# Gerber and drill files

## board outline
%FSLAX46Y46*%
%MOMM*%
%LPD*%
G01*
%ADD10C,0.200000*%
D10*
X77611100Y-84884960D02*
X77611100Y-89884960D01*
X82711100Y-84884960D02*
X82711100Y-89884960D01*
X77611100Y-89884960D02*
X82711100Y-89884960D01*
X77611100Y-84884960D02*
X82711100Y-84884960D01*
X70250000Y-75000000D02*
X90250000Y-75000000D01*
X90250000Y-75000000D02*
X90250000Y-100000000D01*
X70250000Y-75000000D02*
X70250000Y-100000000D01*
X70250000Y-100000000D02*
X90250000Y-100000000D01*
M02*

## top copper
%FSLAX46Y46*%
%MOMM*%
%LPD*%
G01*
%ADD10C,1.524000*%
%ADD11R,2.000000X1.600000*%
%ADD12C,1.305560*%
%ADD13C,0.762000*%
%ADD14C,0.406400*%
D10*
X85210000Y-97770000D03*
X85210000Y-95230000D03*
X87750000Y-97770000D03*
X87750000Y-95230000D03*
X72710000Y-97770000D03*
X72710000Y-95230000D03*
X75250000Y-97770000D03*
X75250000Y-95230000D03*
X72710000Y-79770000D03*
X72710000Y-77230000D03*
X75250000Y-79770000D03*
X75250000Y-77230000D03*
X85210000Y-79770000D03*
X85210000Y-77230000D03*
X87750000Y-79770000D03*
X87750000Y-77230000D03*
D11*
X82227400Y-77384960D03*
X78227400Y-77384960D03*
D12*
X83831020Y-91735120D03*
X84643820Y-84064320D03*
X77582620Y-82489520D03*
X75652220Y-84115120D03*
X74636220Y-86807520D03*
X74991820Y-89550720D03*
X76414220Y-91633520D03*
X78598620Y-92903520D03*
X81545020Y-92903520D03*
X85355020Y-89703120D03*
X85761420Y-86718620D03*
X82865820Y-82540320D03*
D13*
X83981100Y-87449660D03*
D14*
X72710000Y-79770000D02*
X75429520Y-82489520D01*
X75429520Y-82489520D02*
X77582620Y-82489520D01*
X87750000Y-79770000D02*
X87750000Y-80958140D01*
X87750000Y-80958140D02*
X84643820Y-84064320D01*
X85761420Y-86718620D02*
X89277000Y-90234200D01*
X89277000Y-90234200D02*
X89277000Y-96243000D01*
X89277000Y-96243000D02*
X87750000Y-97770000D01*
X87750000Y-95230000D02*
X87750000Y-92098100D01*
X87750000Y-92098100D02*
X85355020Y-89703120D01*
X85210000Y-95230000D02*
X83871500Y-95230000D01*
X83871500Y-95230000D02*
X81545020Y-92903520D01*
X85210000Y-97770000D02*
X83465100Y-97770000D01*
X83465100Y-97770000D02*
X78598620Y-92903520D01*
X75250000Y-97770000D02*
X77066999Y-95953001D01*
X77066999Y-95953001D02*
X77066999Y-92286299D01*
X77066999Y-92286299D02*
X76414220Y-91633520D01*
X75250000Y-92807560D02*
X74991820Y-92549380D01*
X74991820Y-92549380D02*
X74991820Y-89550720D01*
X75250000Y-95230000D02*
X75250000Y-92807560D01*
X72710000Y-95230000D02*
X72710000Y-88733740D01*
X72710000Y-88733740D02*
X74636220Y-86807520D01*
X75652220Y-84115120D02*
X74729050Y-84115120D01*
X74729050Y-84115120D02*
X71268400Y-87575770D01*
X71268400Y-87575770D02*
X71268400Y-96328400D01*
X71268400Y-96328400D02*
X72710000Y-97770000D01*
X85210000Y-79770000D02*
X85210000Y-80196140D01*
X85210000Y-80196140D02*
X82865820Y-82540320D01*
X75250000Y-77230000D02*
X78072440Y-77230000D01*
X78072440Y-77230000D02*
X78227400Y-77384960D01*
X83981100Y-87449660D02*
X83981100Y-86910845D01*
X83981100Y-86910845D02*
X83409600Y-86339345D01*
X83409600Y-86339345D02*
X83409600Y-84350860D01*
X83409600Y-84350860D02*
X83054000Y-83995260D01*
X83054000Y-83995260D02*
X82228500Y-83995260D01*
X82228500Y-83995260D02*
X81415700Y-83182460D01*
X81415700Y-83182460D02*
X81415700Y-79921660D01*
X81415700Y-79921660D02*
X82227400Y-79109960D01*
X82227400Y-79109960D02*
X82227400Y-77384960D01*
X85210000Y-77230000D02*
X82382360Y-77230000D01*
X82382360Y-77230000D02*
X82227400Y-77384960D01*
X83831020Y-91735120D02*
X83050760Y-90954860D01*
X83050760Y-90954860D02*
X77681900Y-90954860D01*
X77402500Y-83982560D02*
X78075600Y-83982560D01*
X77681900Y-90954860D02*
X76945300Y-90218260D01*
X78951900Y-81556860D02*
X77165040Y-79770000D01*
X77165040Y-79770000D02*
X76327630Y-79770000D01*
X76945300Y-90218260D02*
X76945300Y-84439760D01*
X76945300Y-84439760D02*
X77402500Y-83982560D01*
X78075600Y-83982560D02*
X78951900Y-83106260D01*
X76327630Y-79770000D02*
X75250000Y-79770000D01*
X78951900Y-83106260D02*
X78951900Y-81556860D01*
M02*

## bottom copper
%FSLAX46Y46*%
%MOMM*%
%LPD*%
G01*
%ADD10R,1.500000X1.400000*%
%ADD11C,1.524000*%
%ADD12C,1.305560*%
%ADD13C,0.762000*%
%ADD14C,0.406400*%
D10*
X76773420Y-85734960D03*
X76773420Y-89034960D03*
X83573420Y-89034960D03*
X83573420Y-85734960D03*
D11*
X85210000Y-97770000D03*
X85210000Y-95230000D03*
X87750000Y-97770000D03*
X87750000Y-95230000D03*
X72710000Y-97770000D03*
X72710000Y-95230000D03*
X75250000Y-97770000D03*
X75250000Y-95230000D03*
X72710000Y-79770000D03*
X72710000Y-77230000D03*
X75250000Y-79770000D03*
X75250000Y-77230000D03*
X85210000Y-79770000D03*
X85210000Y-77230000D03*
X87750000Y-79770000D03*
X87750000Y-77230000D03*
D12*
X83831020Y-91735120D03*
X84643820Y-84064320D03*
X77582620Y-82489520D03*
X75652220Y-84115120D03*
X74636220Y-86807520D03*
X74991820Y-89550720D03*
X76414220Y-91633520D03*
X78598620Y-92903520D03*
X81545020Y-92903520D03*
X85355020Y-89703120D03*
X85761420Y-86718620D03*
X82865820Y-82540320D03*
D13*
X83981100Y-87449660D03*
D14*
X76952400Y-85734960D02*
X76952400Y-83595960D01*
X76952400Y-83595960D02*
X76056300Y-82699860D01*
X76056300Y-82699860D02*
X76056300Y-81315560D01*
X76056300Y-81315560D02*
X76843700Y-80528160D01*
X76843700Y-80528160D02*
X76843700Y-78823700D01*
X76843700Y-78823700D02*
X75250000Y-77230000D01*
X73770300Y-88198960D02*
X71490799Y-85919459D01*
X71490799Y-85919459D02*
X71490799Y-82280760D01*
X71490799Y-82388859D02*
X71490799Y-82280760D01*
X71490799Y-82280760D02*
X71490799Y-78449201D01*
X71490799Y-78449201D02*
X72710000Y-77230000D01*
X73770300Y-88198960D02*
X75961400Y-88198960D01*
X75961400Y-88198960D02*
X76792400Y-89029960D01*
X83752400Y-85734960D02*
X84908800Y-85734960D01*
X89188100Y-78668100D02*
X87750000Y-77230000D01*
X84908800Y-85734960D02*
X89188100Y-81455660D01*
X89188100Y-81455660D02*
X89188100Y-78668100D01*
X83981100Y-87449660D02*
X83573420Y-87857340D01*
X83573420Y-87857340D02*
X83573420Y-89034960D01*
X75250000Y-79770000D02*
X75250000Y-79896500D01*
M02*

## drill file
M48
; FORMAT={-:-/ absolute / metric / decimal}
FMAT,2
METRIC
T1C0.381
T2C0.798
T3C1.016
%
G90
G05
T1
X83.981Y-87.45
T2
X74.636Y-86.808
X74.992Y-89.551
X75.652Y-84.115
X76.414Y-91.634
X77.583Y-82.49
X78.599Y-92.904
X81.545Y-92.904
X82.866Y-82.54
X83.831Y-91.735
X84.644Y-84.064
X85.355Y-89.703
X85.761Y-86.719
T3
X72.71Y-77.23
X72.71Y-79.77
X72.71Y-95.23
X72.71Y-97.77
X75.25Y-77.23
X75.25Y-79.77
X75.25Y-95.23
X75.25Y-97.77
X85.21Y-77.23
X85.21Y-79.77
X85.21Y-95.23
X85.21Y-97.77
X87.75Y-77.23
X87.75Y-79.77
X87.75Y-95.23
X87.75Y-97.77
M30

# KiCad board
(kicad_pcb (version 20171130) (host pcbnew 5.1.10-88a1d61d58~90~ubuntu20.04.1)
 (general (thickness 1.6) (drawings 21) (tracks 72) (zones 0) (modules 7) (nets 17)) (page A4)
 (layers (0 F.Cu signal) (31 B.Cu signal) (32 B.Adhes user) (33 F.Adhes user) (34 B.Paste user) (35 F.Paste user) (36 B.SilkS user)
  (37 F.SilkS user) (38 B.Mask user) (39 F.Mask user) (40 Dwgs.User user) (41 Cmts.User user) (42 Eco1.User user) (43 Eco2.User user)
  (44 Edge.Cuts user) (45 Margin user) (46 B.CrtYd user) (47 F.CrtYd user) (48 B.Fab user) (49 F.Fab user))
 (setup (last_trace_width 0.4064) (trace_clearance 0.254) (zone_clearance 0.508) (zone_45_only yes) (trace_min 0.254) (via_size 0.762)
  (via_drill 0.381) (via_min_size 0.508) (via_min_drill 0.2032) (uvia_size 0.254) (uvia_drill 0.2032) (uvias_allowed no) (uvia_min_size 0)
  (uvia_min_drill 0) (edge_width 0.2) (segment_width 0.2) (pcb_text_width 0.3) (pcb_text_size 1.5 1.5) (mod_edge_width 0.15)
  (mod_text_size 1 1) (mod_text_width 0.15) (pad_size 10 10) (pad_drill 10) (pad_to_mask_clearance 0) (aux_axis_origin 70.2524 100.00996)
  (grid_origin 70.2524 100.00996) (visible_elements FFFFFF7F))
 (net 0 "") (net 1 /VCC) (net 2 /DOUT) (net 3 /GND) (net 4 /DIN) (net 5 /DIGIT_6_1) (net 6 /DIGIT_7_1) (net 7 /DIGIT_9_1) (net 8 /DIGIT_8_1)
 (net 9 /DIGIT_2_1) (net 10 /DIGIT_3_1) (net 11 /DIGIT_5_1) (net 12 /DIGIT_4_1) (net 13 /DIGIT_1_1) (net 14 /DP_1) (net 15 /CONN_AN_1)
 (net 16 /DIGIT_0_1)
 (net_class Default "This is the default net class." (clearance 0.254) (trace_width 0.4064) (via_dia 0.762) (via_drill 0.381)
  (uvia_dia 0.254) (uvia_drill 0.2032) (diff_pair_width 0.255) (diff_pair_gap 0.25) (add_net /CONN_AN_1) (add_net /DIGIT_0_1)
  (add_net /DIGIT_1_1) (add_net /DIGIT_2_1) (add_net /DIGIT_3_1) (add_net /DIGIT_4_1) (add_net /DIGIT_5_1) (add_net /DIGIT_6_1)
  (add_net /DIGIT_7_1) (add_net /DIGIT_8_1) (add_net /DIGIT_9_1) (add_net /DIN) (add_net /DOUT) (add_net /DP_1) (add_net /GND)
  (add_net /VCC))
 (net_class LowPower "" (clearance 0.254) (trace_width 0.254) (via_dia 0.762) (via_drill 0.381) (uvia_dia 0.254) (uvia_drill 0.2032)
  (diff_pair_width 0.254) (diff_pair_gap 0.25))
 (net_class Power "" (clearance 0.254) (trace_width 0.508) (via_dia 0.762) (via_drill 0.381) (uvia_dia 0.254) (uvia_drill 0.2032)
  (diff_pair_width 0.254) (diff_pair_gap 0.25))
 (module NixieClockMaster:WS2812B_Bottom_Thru (layer F.Cu) (at 80.17342 87.38496 90)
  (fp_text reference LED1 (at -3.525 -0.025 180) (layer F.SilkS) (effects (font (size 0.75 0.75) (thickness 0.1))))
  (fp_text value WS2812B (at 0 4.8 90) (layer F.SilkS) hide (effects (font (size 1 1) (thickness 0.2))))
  (pad 1 smd rect (at 1.65 -3.4 90) (size 1.4 1.5) (layers B.Cu B.Paste B.Mask) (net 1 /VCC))
  (pad 2 smd rect (at -1.65 -3.4 90) (size 1.4 1.5) (layers B.Cu B.Paste B.Mask) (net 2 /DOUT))
  (pad 3 smd rect (at -1.65 3.4 90) (size 1.4 1.5) (layers B.Cu B.Paste B.Mask) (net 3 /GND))
  (pad 4 smd rect (at 1.65 3.4 90) (size 1.4 1.5) (layers B.Cu B.Paste B.Mask) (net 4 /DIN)))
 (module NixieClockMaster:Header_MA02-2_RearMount (layer F.Cu) (at 87.75 96.5)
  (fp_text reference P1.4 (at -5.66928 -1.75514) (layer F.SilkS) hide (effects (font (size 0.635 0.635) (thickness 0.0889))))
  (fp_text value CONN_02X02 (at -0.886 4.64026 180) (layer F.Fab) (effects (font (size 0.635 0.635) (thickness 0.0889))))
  (pad 1 thru_hole circle (at -2.54 1.27) (size 1.524 1.524) (drill 1.016) (layers *.Cu *.Mask F.Paste F.SilkS) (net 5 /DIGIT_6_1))
  (pad 2 thru_hole circle (at -2.54 -1.27) (size 1.524 1.524) (drill 1.016) (layers *.Cu *.Mask F.Paste F.SilkS) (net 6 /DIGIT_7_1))
  (pad 3 thru_hole circle (at 0 1.27) (size 1.524 1.524) (drill 1.016) (layers *.Cu *.Mask F.Paste F.SilkS) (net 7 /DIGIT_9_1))
  (pad 4 thru_hole circle (at 0 -1.27) (size 1.524 1.524) (drill 1.016) (layers *.Cu *.Mask F.Paste F.SilkS) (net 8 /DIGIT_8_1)))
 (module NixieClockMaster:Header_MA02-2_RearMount (layer F.Cu) (at 75.25 96.5)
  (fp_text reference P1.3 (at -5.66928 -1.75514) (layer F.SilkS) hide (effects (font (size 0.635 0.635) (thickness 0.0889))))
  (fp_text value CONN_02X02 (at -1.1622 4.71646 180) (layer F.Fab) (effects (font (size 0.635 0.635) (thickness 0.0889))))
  (pad 1 thru_hole circle (at -2.54 1.27) (size 1.524 1.524) (drill 1.016) (layers *.Cu *.Mask F.Paste F.SilkS) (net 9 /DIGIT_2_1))
  (pad 2 thru_hole circle (at -2.54 -1.27) (size 1.524 1.524) (drill 1.016) (layers *.Cu *.Mask F.Paste F.SilkS) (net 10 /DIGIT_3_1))
  (pad 3 thru_hole circle (at 0 1.27) (size 1.524 1.524) (drill 1.016) (layers *.Cu *.Mask F.Paste F.SilkS) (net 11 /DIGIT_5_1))
  (pad 4 thru_hole circle (at 0 -1.27) (size 1.524 1.524) (drill 1.016) (layers *.Cu *.Mask F.Paste F.SilkS) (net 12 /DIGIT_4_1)))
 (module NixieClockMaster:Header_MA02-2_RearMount (layer F.Cu) (at 75.25 78.5)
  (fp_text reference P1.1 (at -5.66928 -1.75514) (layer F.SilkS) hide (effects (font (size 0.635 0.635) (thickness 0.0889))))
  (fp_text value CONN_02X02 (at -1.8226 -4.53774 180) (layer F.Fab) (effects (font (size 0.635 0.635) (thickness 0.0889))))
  (pad 1 thru_hole circle (at -2.54 1.27) (size 1.524 1.524) (drill 1.016) (layers *.Cu *.Mask F.Paste F.SilkS) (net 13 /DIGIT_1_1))
  (pad 2 thru_hole circle (at -2.54 -1.27) (size 1.524 1.524) (drill 1.016) (layers *.Cu *.Mask F.Paste F.SilkS) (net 2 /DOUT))
  (pad 3 thru_hole circle (at 0 1.27) (size 1.524 1.524) (drill 1.016) (layers *.Cu *.Mask F.Paste F.SilkS) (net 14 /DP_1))
  (pad 4 thru_hole circle (at 0 -1.27) (size 1.524 1.524) (drill 1.016) (layers *.Cu *.Mask F.Paste F.SilkS) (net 1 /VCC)))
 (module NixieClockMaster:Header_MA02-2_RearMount (layer F.Cu) (at 87.75 78.5)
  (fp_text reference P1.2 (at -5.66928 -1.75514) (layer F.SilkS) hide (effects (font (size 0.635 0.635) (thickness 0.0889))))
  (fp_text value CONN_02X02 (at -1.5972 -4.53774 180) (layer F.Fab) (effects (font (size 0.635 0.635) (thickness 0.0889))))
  (pad 1 thru_hole circle (at -2.54 1.27) (size 1.524 1.524) (drill 1.016) (layers *.Cu *.Mask F.Paste F.SilkS) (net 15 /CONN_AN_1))
  (pad 2 thru_hole circle (at -2.54 -1.27) (size 1.524 1.524) (drill 1.016) (layers *.Cu *.Mask F.Paste F.SilkS) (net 3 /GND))
  (pad 3 thru_hole circle (at 0 1.27) (size 1.524 1.524) (drill 1.016) (layers *.Cu *.Mask F.Paste F.SilkS) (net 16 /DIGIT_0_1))
  (pad 4 thru_hole circle (at 0 -1.27) (size 1.524 1.524) (drill 1.016) (layers *.Cu *.Mask F.Paste F.SilkS) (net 4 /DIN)))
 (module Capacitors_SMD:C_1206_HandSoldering (layer F.Cu) (at 80.2274 77.38496 180)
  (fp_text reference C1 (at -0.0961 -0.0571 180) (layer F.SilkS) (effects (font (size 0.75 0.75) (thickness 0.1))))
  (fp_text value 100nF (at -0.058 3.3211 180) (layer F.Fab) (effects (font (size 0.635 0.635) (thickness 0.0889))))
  (pad 1 smd rect (at -2 0 180) (size 2 1.6) (layers F.Cu F.Paste F.Mask) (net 3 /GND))
  (pad 2 smd rect (at 2 0 180) (size 2 1.6) (layers F.Cu F.Paste F.Mask) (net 1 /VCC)))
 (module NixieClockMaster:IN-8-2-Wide (layer F.Cu) (at 80.17342 87.46792 180)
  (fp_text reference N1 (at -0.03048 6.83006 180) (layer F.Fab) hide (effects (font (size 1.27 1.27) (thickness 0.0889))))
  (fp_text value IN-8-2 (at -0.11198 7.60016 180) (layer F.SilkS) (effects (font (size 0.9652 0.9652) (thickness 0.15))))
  (pad . thru_hole circle (at -3.6576 -4.2672 180) (size 1.30556 1.30556) (drill 0.79756) (layers *.Cu *.Mask F.Paste F.SilkS)
   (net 14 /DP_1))
  (pad 0 thru_hole circle (at -4.4704 3.4036 180) (size 1.30556 1.30556) (drill 0.79756) (layers *.Cu *.Mask F.Paste F.SilkS)
   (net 16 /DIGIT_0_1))
  (pad 1 thru_hole circle (at 2.5908 4.9784 180) (size 1.30556 1.30556) (drill 0.79756) (layers *.Cu *.Mask F.Paste F.SilkS)
   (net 13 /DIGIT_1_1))
  (pad 2 thru_hole circle (at 4.5212 3.3528 180) (size 1.30556 1.30556) (drill 0.79756) (layers *.Cu *.Mask F.Paste F.SilkS)
   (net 9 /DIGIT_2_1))
  (pad 3 thru_hole circle (at 5.5372 0.6604 180) (size 1.30556 1.30556) (drill 0.79756) (layers *.Cu *.Mask F.Paste F.SilkS)
   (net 10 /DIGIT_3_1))
  (pad 4 thru_hole circle (at 5.1816 -2.0828 180) (size 1.30556 1.30556) (drill 0.79756) (layers *.Cu *.Mask F.Paste F.SilkS)
   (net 12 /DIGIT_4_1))
  (pad 5 thru_hole circle (at 3.7592 -4.1656 180) (size 1.30556 1.30556) (drill 0.79756) (layers *.Cu *.Mask F.Paste F.SilkS)
   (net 11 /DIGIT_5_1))
  (pad 6 thru_hole circle (at 1.5748 -5.4356 180) (size 1.30556 1.30556) (drill 0.79756) (layers *.Cu *.Mask F.Paste F.SilkS)
   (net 5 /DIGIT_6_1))
  (pad 7 thru_hole circle (at -1.3716 -5.4356 180) (size 1.30556 1.30556) (drill 0.79756) (layers *.Cu *.Mask F.Paste F.SilkS)
   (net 6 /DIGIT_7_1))
  (pad 8 thru_hole circle (at -5.1816 -2.2352 180) (size 1.30556 1.30556) (drill 0.79756) (layers *.Cu *.Mask F.Paste F.SilkS)
   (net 8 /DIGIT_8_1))
  (pad 9 thru_hole circle (at -5.588 0.7493 180) (size 1.30556 1.30556) (drill 0.79756) (layers *.Cu *.Mask F.Paste F.SilkS)
   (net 7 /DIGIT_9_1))
  (pad A thru_hole circle (at -2.6924 4.9276 180) (size 1.30556 1.30556) (drill 0.79756) (layers *.Cu *.Mask F.Paste F.SilkS)
   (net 15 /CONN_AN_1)))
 (gr_line (start 77.6111 84.88496) (end 77.6111 89.88496) (layer Edge.Cuts) (width 0.2))
 (gr_line (start 82.7111 84.88496) (end 82.7111 89.88496) (layer Edge.Cuts) (width 0.2))
 (gr_line (start 77.6111 89.88496) (end 82.7111 89.88496) (layer Edge.Cuts) (width 0.2))
 (gr_line (start 77.6111 84.88496) (end 82.7111 84.88496) (layer Edge.Cuts) (width 0.2))
 (gr_line (start 70.25 75) (end 90.25 75) (layer Edge.Cuts) (width 0.2))
 (gr_line (start 90.25 75) (end 90.25 100) (layer Edge.Cuts) (width 0.2))
 (gr_line (start 70.25 75) (end 70.25 100) (layer Edge.Cuts) (width 0.2))
 (gr_line (start 70.25 100) (end 90.25 100) (layer Edge.Cuts) (width 0.2))
 (segment (start 72.71 79.77) (end 75.42952 82.48952) (width 0.4064) (layer F.Cu) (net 13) (status 10))
 (segment (start 75.42952 82.48952) (end 77.58262 82.48952) (width 0.4064) (layer F.Cu) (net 13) (status 20))
 (segment (start 87.75 79.77) (end 87.75 80.95814) (width 0.4064) (layer F.Cu) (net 16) (status 10))
 (segment (start 87.75 80.95814) (end 84.64382 84.06432) (width 0.4064) (layer F.Cu) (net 16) (status 20))
 (segment (start 85.76142 86.71862) (end 89.277 90.2342) (width 0.4064) (layer F.Cu) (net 7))
 (segment (start 89.277 90.2342) (end 89.277 96.243) (width 0.4064) (layer F.Cu) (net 7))
 (segment (start 89.277 96.243) (end 87.75 97.77) (width 0.4064) (layer F.Cu) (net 7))
 (segment (start 87.75 95.23) (end 87.75 92.0981) (width 0.4064) (layer F.Cu) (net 8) (status 10))
 (segment (start 87.75 92.0981) (end 85.35502 89.70312) (width 0.4064) (layer F.Cu) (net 8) (status 20))
 (segment (start 85.21 95.23) (end 83.8715 95.23) (width 0.4064) (layer F.Cu) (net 6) (status 10))
 (segment (start 83.8715 95.23) (end 81.54502 92.90352) (width 0.4064) (layer F.Cu) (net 6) (status 20))
 (segment (start 85.21 97.77) (end 83.4651 97.77) (width 0.4064) (layer F.Cu) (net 5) (status 10))
 (segment (start 83.4651 97.77) (end 78.59862 92.90352) (width 0.4064) (layer F.Cu) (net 5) (status 20))
 (segment (start 75.25 97.77) (end 77.066999 95.953001) (width 0.4064) (layer F.Cu) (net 11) (status 10))
 (segment (start 77.066999 95.953001) (end 77.066999 92.286299) (width 0.4064) (layer F.Cu) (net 11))
 (segment (start 77.066999 92.286299) (end 76.41422 91.63352) (width 0.4064) (layer F.Cu) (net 11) (status 20))
 (segment (start 75.25 92.80756) (end 74.99182 92.54938) (width 0.4064) (layer F.Cu) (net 12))
 (segment (start 74.99182 92.54938) (end 74.99182 89.55072) (width 0.4064) (layer F.Cu) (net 12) (status 20))
 (segment (start 75.25 95.23) (end 75.25 92.80756) (width 0.4064) (layer F.Cu) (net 12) (status 10))
 (segment (start 72.71 95.23) (end 72.71 88.73374) (width 0.4064) (layer F.Cu) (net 10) (status 10))
 (segment (start 72.71 88.73374) (end 74.63622 86.80752) (width 0.4064) (layer F.Cu) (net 10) (status 20))
 (segment (start 75.65222 84.11512) (end 74.72905 84.11512) (width 0.4064) (layer F.Cu) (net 9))
 (segment (start 74.72905 84.11512) (end 71.2684 87.57577) (width 0.4064) (layer F.Cu) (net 9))
 (segment (start 71.2684 87.57577) (end 71.2684 96.3284) (width 0.4064) (layer F.Cu) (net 9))
 (segment (start 71.2684 96.3284) (end 72.71 97.77) (width 0.4064) (layer F.Cu) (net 9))
 (segment (start 85.21 79.77) (end 85.21 80.19614) (width 0.4064) (layer F.Cu) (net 15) (status 30))
 (segment (start 85.21 80.19614) (end 82.86582 82.54032) (width 0.4064) (layer F.Cu) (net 15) (status 30))
 (segment (start 76.9524 85.73496) (end 76.9524 83.59596) (width 0.4064) (layer B.Cu) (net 1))
 (segment (start 76.9524 83.59596) (end 76.0563 82.69986) (width 0.4064) (layer B.Cu) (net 1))
 (segment (start 76.0563 82.69986) (end 76.0563 81.31556) (width 0.4064) (layer B.Cu) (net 1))
 (segment (start 76.0563 81.31556) (end 76.8437 80.52816) (width 0.4064) (layer B.Cu) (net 1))
 (segment (start 76.8437 80.52816) (end 76.8437 78.8237) (width 0.4064) (layer B.Cu) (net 1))
 (segment (start 76.8437 78.8237) (end 75.25 77.23) (width 0.4064) (layer B.Cu) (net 1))
 (segment (start 75.25 77.23) (end 78.07244 77.23) (width 0.4064) (layer F.Cu) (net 1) (status 30))
 (segment (start 78.07244 77.23) (end 78.2274 77.38496) (width 0.4064) (layer F.Cu) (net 1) (status 30))
 (segment (start 73.7703 88.19896) (end 71.490799 85.919459) (width 0.4064) (layer B.Cu) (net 2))
 (segment (start 71.490799 85.919459) (end 71.490799 82.28076) (width 0.4064) (layer B.Cu) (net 2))
 (segment (start 71.490799 82.388859) (end 71.490799 82.28076) (width 0.4064) (layer B.Cu) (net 2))
 (segment (start 71.490799 82.28076) (end 71.490799 78.449201) (width 0.4064) (layer B.Cu) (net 2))
 (segment (start 71.490799 78.449201) (end 72.71 77.23) (width 0.4064) (layer B.Cu) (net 2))
 (segment (start 73.7703 88.19896) (end 75.9614 88.19896) (width 0.4064) (layer B.Cu) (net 2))
 (segment (start 75.9614 88.19896) (end 76.7924 89.02996) (width 0.4064) (layer B.Cu) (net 2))
 (segment (start 83.7524 85.73496) (end 84.9088 85.73496) (width 0.4064) (layer B.Cu) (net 4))
 (segment (start 89.1881 78.6681) (end 87.75 77.23) (width 0.4064) (layer B.Cu) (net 4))
 (segment (start 84.9088 85.73496) (end 89.1881 81.45566) (width 0.4064) (layer B.Cu) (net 4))
 (segment (start 89.1881 81.45566) (end 89.1881 78.6681) (width 0.4064) (layer B.Cu) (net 4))
 (segment (start 83.9811 87.44966) (end 83.9811 86.910845) (width 0.4064) (layer F.Cu) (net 3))
 (segment (start 83.9811 86.910845) (end 83.4096 86.339345) (width 0.4064) (layer F.Cu) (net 3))
 (segment (start 83.4096 86.339345) (end 83.4096 84.35086) (width 0.4064) (layer F.Cu) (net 3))
 (segment (start 83.4096 84.35086) (end 83.054 83.99526) (width 0.4064) (layer F.Cu) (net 3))
 (segment (start 83.054 83.99526) (end 82.2285 83.99526) (width 0.4064) (layer F.Cu) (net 3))
 (segment (start 82.2285 83.99526) (end 81.4157 83.18246) (width 0.4064) (layer F.Cu) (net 3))
 (segment (start 81.4157 83.18246) (end 81.4157 79.92166) (width 0.4064) (layer F.Cu) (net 3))
 (segment (start 81.4157 79.92166) (end 82.2274 79.10996) (width 0.4064) (layer F.Cu) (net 3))
 (segment (start 82.2274 79.10996) (end 82.2274 77.38496) (width 0.4064) (layer F.Cu) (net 3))
 (segment (start 83.9811 87.44966) (end 83.57342 87.85734) (width 0.4064) (layer B.Cu) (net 3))
 (segment (start 83.57342 87.85734) (end 83.57342 89.03496) (width 0.4064) (layer B.Cu) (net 3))
 (via (at 83.9811 87.44966) (size 0.762) (drill 0.381) (layers F.Cu B.Cu) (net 3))
 (segment (start 85.21 77.23) (end 82.38236 77.23) (width 0.4064) (layer F.Cu) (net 3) (status 30))
 (segment (start 82.38236 77.23) (end 82.2274 77.38496) (width 0.4064) (layer F.Cu) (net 3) (status 30))
 (segment (start 83.83102 91.73512) (end 83.05076 90.95486) (width 0.4064) (layer F.Cu) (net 14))
 (segment (start 83.05076 90.95486) (end 77.6819 90.95486) (width 0.4064) (layer F.Cu) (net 14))
 (segment (start 77.4025 83.98256) (end 78.0756 83.98256) (width 0.4064) (layer F.Cu) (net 14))
 (segment (start 77.6819 90.95486) (end 76.9453 90.21826) (width 0.4064) (layer F.Cu) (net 14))
 (segment (start 78.9519 81.55686) (end 77.16504 79.77) (width 0.4064) (layer F.Cu) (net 14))
 (segment (start 77.16504 79.77) (end 76.32763 79.77) (width 0.4064) (layer F.Cu) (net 14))
 (segment (start 76.9453 90.21826) (end 76.9453 84.43976) (width 0.4064) (layer F.Cu) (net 14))
 (segment (start 76.9453 84.43976) (end 77.4025 83.98256) (width 0.4064) (layer F.Cu) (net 14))
 (segment (start 78.0756 83.98256) (end 78.9519 83.10626) (width 0.4064) (layer F.Cu) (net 14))
 (segment (start 76.32763 79.77) (end 75.25 79.77) (width 0.4064) (layer F.Cu) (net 14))
 (segment (start 78.9519 83.10626) (end 78.9519 81.55686) (width 0.4064) (layer F.Cu) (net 14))
 (segment (start 75.25 79.77) (end 75.25 79.8965) (width 0.4064) (layer B.Cu) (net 14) (status 30))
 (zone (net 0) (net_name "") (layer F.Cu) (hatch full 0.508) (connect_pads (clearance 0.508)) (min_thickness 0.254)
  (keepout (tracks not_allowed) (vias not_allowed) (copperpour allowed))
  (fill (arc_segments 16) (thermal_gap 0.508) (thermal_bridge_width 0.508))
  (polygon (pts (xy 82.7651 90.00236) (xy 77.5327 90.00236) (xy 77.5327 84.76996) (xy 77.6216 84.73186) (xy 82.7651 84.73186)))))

